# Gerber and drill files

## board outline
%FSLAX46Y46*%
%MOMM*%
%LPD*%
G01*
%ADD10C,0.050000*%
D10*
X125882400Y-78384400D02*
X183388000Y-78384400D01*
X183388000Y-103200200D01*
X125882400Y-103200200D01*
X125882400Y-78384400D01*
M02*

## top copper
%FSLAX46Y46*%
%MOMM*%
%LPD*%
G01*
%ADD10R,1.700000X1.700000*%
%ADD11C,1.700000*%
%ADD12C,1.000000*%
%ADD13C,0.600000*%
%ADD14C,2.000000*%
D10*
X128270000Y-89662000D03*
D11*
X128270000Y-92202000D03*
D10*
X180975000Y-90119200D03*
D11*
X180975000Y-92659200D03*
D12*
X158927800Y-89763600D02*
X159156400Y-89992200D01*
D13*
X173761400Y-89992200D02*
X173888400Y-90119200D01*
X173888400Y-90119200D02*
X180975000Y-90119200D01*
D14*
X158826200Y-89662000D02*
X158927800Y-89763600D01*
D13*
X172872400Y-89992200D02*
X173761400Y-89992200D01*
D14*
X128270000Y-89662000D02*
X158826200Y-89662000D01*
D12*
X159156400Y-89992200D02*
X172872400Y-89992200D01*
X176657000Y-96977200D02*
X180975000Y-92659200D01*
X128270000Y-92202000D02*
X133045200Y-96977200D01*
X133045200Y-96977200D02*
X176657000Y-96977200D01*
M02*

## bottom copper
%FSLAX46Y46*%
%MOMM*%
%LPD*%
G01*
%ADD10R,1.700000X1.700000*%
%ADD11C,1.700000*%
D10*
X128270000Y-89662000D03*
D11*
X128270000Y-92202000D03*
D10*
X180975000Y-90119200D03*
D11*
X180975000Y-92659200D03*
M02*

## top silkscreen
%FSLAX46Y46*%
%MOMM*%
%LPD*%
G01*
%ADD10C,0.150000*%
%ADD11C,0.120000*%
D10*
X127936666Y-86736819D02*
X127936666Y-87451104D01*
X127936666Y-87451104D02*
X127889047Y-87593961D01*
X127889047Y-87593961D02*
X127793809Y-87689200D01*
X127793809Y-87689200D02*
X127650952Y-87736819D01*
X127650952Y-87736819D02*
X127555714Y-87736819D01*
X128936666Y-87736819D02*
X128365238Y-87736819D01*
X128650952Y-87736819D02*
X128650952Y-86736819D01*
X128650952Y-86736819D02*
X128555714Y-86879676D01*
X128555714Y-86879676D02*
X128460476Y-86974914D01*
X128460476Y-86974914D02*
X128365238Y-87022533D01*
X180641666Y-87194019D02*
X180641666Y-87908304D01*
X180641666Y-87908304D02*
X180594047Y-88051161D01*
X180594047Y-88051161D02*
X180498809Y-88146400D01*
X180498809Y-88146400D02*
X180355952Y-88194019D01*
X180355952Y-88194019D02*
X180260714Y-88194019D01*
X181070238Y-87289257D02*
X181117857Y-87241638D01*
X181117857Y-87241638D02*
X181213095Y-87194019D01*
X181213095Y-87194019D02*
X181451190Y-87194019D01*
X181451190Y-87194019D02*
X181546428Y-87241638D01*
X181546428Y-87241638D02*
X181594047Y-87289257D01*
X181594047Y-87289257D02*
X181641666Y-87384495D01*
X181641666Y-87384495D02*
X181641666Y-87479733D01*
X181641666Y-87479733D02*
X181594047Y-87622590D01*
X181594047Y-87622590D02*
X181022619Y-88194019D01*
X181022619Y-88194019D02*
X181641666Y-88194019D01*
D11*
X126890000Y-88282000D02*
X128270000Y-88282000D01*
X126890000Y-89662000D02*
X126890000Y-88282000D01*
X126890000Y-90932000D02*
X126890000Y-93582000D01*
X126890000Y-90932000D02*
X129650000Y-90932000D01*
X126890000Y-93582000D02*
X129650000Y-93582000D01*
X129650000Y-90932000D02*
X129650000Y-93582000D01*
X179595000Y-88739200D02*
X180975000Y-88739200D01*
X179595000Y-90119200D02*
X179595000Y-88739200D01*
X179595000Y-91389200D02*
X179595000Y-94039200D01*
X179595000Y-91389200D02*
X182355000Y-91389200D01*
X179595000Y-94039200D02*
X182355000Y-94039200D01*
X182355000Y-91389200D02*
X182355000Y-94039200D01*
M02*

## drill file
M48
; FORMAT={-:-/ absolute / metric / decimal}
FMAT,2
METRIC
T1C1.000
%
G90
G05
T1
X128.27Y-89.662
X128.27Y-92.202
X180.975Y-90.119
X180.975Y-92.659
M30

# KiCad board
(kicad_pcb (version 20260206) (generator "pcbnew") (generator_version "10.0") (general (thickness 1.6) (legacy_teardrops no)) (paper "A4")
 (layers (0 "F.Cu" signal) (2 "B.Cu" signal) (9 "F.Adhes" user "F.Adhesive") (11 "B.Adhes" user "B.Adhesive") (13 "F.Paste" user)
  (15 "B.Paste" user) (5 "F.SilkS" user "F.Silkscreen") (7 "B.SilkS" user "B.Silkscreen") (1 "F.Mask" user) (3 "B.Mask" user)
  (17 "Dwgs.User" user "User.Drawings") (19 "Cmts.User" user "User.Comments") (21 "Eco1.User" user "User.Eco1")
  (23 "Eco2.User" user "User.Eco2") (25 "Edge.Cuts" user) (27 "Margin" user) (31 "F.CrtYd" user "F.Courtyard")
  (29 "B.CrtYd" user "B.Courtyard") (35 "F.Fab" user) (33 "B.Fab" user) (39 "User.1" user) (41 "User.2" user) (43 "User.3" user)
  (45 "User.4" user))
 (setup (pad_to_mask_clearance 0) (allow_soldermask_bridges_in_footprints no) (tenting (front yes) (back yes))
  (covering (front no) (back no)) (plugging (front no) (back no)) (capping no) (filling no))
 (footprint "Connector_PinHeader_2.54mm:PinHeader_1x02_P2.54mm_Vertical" (layer "F.Cu") (at 128.27 89.662)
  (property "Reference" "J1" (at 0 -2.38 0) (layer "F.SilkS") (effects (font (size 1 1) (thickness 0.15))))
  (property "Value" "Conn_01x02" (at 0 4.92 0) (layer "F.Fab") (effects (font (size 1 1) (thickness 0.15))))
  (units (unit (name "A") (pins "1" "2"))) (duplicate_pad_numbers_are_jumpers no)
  (fp_line (start -1.38 -1.38) (end 0 -1.38) (stroke (width 0.12) (type solid)) (layer "F.SilkS"))
  (fp_line (start -1.38 0) (end -1.38 -1.38) (stroke (width 0.12) (type solid)) (layer "F.SilkS"))
  (fp_line (start -1.38 1.27) (end -1.38 3.92) (stroke (width 0.12) (type solid)) (layer "F.SilkS"))
  (fp_line (start -1.38 1.27) (end 1.38 1.27) (stroke (width 0.12) (type solid)) (layer "F.SilkS"))
  (fp_line (start -1.38 3.92) (end 1.38 3.92) (stroke (width 0.12) (type solid)) (layer "F.SilkS"))
  (fp_line (start 1.38 1.27) (end 1.38 3.92) (stroke (width 0.12) (type solid)) (layer "F.SilkS"))
  (pad "1" thru_hole rect (at 0 0) (size 1.7 1.7) (drill 1) (layers "*.Cu" "*.Mask") (remove_unused_layers no) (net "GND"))
  (pad "2" thru_hole circle (at 0 2.54) (size 1.7 1.7) (drill 1) (layers "*.Cu" "*.Mask") (remove_unused_layers no) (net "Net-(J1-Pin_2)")))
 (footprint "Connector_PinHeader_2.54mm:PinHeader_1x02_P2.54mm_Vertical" (layer "F.Cu") (at 180.975 90.1192)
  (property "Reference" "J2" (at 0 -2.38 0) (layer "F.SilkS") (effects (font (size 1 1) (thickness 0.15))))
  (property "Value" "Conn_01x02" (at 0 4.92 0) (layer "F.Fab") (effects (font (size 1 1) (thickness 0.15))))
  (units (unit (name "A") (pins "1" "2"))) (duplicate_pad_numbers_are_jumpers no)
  (fp_line (start -1.38 -1.38) (end 0 -1.38) (stroke (width 0.12) (type solid)) (layer "F.SilkS"))
  (fp_line (start -1.38 0) (end -1.38 -1.38) (stroke (width 0.12) (type solid)) (layer "F.SilkS"))
  (fp_line (start -1.38 1.27) (end -1.38 3.92) (stroke (width 0.12) (type solid)) (layer "F.SilkS"))
  (fp_line (start -1.38 1.27) (end 1.38 1.27) (stroke (width 0.12) (type solid)) (layer "F.SilkS"))
  (fp_line (start -1.38 3.92) (end 1.38 3.92) (stroke (width 0.12) (type solid)) (layer "F.SilkS"))
  (fp_line (start 1.38 1.27) (end 1.38 3.92) (stroke (width 0.12) (type solid)) (layer "F.SilkS"))
  (pad "1" thru_hole rect (at 0 0) (size 1.7 1.7) (drill 1) (layers "*.Cu" "*.Mask") (remove_unused_layers no) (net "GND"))
  (pad "2" thru_hole circle (at 0 2.54) (size 1.7 1.7) (drill 1) (layers "*.Cu" "*.Mask") (remove_unused_layers no) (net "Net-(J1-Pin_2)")))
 (gr_rect (start 125.8824 78.3844) (end 183.388 103.2002) (stroke (width 0.05) (type default)) (fill no) (layer "Edge.Cuts"))
 (segment (start 158.9278 89.7636) (end 159.1564 89.9922) (width 1) (layer "F.Cu") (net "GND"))
 (segment (start 173.7614 89.9922) (end 173.8884 90.1192) (width 0.6) (layer "F.Cu") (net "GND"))
 (segment (start 173.8884 90.1192) (end 180.975 90.1192) (width 0.6) (layer "F.Cu") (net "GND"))
 (segment (start 158.8262 89.662) (end 158.9278 89.7636) (width 2) (layer "F.Cu") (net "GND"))
 (segment (start 172.8724 89.9922) (end 173.7614 89.9922) (width 0.6) (layer "F.Cu") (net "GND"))
 (segment (start 128.27 89.662) (end 158.8262 89.662) (width 2) (layer "F.Cu") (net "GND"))
 (segment (start 159.1564 89.9922) (end 172.8724 89.9922) (width 1) (layer "F.Cu") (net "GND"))
 (segment (start 176.657 96.9772) (end 180.975 92.6592) (width 1) (layer "F.Cu") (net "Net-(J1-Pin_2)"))
 (segment (start 128.27 92.202) (end 133.0452 96.9772) (width 1) (layer "F.Cu") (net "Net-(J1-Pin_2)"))
 (segment (start 133.0452 96.9772) (end 176.657 96.9772) (width 1) (layer "F.Cu") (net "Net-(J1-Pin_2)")))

